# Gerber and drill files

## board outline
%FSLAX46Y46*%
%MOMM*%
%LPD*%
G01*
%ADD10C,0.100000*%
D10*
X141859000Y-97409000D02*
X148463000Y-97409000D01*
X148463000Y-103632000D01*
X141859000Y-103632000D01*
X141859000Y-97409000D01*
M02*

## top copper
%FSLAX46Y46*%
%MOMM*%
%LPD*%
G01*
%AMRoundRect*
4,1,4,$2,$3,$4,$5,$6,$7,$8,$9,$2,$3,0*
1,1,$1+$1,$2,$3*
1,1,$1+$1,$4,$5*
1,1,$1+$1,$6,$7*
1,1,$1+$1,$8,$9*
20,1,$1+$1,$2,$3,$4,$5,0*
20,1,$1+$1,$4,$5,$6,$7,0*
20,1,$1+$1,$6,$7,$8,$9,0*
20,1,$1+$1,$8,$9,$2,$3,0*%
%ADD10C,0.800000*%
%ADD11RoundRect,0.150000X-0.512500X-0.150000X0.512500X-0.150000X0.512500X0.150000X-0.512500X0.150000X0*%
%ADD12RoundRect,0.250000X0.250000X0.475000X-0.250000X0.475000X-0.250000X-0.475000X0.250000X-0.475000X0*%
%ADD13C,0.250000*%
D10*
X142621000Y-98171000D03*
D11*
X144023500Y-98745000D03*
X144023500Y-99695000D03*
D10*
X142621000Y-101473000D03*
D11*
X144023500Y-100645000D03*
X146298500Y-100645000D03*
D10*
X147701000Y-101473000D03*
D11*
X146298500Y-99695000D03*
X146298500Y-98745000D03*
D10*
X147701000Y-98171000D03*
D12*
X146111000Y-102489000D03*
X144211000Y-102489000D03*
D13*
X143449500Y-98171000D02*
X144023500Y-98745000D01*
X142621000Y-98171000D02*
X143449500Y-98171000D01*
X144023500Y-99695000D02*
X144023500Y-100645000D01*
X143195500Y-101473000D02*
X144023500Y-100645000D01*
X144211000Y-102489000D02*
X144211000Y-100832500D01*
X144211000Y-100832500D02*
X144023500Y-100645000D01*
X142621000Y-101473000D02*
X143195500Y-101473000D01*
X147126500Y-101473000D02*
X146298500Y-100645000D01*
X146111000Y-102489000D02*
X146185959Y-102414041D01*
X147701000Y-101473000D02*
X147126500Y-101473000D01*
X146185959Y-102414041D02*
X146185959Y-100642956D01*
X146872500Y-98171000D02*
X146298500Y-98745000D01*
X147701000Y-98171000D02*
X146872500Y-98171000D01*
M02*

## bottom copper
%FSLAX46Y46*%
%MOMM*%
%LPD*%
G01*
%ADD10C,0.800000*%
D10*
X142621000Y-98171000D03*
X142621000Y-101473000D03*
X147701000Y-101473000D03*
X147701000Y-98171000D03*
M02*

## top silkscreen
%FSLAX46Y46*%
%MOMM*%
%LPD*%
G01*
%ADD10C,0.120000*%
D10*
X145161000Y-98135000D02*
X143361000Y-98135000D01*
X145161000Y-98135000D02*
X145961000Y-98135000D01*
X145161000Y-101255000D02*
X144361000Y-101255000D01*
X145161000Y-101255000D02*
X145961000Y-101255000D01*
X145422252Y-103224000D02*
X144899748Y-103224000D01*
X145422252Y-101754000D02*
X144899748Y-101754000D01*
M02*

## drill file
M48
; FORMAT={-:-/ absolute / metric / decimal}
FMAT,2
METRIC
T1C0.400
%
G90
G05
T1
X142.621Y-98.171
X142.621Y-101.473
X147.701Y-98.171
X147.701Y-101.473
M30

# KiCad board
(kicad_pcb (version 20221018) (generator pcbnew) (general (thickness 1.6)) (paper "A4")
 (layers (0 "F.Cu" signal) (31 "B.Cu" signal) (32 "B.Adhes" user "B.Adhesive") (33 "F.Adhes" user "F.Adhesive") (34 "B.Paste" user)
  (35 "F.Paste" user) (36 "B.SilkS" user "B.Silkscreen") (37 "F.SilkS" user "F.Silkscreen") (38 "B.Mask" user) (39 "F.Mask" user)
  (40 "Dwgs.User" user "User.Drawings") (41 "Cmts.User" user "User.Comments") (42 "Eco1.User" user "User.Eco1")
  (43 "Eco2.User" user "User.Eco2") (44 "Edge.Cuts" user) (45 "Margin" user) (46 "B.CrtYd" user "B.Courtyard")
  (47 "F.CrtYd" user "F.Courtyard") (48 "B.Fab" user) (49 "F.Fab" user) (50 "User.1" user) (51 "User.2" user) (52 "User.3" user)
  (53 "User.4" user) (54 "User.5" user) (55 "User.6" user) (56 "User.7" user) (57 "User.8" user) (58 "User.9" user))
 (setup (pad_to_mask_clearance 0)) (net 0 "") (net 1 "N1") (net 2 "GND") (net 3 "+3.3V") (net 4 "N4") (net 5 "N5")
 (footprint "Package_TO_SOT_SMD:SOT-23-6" (layer "F.Cu") (at 145.161 99.695)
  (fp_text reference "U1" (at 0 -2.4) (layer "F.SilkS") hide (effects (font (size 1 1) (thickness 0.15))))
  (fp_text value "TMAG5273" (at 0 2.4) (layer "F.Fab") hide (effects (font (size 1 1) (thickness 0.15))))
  (fp_line (start 0 -1.56) (end -1.8 -1.56) (stroke (width 0.12) (type solid)) (layer "F.SilkS"))
  (fp_line (start 0 -1.56) (end 0.8 -1.56) (stroke (width 0.12) (type solid)) (layer "F.SilkS"))
  (fp_line (start 0 1.56) (end -0.8 1.56) (stroke (width 0.12) (type solid)) (layer "F.SilkS"))
  (fp_line (start 0 1.56) (end 0.8 1.56) (stroke (width 0.12) (type solid)) (layer "F.SilkS"))
  (pad "1" thru_hole circle (at -2.54 -1.524) (size 0.8 0.8) (drill 0.4) (layers "*.Cu" "*.Mask") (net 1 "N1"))
  (pad "1" smd roundrect (at -1.1375 -0.95) (size 1.325 0.6) (layers "F.Cu" "F.Paste" "F.Mask") (roundrect_rratio 0.25) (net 1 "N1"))
  (pad "2" smd roundrect (at -1.1375 0) (size 1.325 0.6) (layers "F.Cu" "F.Paste" "F.Mask") (roundrect_rratio 0.25) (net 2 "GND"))
  (pad "3" thru_hole circle (at -2.54 1.778) (size 0.8 0.8) (drill 0.4) (layers "*.Cu" "*.Mask") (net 2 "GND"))
  (pad "3" smd roundrect (at -1.1375 0.95) (size 1.325 0.6) (layers "F.Cu" "F.Paste" "F.Mask") (roundrect_rratio 0.25) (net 2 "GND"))
  (pad "4" smd roundrect (at 1.1375 0.95) (size 1.325 0.6) (layers "F.Cu" "F.Paste" "F.Mask") (roundrect_rratio 0.25) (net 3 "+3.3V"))
  (pad "4" thru_hole circle (at 2.54 1.778) (size 0.8 0.8) (drill 0.4) (layers "*.Cu" "*.Mask") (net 3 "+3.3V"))
  (pad "5" smd roundrect (at 1.1375 0) (size 1.325 0.6) (layers "F.Cu" "F.Paste" "F.Mask") (roundrect_rratio 0.25) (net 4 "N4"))
  (pad "6" smd roundrect (at 1.1375 -0.95) (size 1.325 0.6) (layers "F.Cu" "F.Paste" "F.Mask") (roundrect_rratio 0.25) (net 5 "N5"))
  (pad "6" thru_hole circle (at 2.54 -1.524) (size 0.8 0.8) (drill 0.4) (layers "*.Cu" "*.Mask") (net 5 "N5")))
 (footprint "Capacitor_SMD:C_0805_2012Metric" (layer "F.Cu") (at 145.161 102.489 180)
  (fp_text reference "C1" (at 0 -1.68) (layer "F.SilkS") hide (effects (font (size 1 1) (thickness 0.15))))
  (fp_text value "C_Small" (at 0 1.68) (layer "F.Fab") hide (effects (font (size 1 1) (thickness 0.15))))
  (fp_line (start -0.261252 -0.735) (end 0.261252 -0.735) (stroke (width 0.12) (type solid)) (layer "F.SilkS"))
  (fp_line (start -0.261252 0.735) (end 0.261252 0.735) (stroke (width 0.12) (type solid)) (layer "F.SilkS"))
  (pad "1" smd roundrect (at -0.95 0 180) (size 1 1.45) (layers "F.Cu" "F.Paste" "F.Mask") (roundrect_rratio 0.25) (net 3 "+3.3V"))
  (pad "2" smd roundrect (at 0.95 0 180) (size 1 1.45) (layers "F.Cu" "F.Paste" "F.Mask") (roundrect_rratio 0.25) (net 2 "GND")))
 (gr_rect (start 141.859 97.409) (end 148.463 103.632) (stroke (width 0.1) (type solid)) (fill none) (layer "Edge.Cuts"))
 (segment (start 143.4495 98.171) (end 144.0235 98.745) (width 0.25) (layer "F.Cu") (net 1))
 (segment (start 142.621 98.171) (end 143.4495 98.171) (width 0.25) (layer "F.Cu") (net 1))
 (segment (start 144.0235 99.695) (end 144.0235 100.645) (width 0.25) (layer "F.Cu") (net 2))
 (segment (start 143.1955 101.473) (end 144.0235 100.645) (width 0.25) (layer "F.Cu") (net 2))
 (segment (start 144.211 102.489) (end 144.211 100.8325) (width 0.25) (layer "F.Cu") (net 2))
 (segment (start 144.211 100.8325) (end 144.0235 100.645) (width 0.25) (layer "F.Cu") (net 2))
 (segment (start 142.621 101.473) (end 143.1955 101.473) (width 0.25) (layer "F.Cu") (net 2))
 (segment (start 147.1265 101.473) (end 146.2985 100.645) (width 0.25) (layer "F.Cu") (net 3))
 (segment (start 146.111 102.489) (end 146.185959 102.414041) (width 0.25) (layer "F.Cu") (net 3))
 (segment (start 147.701 101.473) (end 147.1265 101.473) (width 0.25) (layer "F.Cu") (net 3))
 (segment (start 146.185959 102.414041) (end 146.185959 100.642956) (width 0.25) (layer "F.Cu") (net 3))
 (segment (start 146.8725 98.171) (end 146.2985 98.745) (width 0.25) (layer "F.Cu") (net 5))
 (segment (start 147.701 98.171) (end 146.8725 98.171) (width 0.25) (layer "F.Cu") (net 5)))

